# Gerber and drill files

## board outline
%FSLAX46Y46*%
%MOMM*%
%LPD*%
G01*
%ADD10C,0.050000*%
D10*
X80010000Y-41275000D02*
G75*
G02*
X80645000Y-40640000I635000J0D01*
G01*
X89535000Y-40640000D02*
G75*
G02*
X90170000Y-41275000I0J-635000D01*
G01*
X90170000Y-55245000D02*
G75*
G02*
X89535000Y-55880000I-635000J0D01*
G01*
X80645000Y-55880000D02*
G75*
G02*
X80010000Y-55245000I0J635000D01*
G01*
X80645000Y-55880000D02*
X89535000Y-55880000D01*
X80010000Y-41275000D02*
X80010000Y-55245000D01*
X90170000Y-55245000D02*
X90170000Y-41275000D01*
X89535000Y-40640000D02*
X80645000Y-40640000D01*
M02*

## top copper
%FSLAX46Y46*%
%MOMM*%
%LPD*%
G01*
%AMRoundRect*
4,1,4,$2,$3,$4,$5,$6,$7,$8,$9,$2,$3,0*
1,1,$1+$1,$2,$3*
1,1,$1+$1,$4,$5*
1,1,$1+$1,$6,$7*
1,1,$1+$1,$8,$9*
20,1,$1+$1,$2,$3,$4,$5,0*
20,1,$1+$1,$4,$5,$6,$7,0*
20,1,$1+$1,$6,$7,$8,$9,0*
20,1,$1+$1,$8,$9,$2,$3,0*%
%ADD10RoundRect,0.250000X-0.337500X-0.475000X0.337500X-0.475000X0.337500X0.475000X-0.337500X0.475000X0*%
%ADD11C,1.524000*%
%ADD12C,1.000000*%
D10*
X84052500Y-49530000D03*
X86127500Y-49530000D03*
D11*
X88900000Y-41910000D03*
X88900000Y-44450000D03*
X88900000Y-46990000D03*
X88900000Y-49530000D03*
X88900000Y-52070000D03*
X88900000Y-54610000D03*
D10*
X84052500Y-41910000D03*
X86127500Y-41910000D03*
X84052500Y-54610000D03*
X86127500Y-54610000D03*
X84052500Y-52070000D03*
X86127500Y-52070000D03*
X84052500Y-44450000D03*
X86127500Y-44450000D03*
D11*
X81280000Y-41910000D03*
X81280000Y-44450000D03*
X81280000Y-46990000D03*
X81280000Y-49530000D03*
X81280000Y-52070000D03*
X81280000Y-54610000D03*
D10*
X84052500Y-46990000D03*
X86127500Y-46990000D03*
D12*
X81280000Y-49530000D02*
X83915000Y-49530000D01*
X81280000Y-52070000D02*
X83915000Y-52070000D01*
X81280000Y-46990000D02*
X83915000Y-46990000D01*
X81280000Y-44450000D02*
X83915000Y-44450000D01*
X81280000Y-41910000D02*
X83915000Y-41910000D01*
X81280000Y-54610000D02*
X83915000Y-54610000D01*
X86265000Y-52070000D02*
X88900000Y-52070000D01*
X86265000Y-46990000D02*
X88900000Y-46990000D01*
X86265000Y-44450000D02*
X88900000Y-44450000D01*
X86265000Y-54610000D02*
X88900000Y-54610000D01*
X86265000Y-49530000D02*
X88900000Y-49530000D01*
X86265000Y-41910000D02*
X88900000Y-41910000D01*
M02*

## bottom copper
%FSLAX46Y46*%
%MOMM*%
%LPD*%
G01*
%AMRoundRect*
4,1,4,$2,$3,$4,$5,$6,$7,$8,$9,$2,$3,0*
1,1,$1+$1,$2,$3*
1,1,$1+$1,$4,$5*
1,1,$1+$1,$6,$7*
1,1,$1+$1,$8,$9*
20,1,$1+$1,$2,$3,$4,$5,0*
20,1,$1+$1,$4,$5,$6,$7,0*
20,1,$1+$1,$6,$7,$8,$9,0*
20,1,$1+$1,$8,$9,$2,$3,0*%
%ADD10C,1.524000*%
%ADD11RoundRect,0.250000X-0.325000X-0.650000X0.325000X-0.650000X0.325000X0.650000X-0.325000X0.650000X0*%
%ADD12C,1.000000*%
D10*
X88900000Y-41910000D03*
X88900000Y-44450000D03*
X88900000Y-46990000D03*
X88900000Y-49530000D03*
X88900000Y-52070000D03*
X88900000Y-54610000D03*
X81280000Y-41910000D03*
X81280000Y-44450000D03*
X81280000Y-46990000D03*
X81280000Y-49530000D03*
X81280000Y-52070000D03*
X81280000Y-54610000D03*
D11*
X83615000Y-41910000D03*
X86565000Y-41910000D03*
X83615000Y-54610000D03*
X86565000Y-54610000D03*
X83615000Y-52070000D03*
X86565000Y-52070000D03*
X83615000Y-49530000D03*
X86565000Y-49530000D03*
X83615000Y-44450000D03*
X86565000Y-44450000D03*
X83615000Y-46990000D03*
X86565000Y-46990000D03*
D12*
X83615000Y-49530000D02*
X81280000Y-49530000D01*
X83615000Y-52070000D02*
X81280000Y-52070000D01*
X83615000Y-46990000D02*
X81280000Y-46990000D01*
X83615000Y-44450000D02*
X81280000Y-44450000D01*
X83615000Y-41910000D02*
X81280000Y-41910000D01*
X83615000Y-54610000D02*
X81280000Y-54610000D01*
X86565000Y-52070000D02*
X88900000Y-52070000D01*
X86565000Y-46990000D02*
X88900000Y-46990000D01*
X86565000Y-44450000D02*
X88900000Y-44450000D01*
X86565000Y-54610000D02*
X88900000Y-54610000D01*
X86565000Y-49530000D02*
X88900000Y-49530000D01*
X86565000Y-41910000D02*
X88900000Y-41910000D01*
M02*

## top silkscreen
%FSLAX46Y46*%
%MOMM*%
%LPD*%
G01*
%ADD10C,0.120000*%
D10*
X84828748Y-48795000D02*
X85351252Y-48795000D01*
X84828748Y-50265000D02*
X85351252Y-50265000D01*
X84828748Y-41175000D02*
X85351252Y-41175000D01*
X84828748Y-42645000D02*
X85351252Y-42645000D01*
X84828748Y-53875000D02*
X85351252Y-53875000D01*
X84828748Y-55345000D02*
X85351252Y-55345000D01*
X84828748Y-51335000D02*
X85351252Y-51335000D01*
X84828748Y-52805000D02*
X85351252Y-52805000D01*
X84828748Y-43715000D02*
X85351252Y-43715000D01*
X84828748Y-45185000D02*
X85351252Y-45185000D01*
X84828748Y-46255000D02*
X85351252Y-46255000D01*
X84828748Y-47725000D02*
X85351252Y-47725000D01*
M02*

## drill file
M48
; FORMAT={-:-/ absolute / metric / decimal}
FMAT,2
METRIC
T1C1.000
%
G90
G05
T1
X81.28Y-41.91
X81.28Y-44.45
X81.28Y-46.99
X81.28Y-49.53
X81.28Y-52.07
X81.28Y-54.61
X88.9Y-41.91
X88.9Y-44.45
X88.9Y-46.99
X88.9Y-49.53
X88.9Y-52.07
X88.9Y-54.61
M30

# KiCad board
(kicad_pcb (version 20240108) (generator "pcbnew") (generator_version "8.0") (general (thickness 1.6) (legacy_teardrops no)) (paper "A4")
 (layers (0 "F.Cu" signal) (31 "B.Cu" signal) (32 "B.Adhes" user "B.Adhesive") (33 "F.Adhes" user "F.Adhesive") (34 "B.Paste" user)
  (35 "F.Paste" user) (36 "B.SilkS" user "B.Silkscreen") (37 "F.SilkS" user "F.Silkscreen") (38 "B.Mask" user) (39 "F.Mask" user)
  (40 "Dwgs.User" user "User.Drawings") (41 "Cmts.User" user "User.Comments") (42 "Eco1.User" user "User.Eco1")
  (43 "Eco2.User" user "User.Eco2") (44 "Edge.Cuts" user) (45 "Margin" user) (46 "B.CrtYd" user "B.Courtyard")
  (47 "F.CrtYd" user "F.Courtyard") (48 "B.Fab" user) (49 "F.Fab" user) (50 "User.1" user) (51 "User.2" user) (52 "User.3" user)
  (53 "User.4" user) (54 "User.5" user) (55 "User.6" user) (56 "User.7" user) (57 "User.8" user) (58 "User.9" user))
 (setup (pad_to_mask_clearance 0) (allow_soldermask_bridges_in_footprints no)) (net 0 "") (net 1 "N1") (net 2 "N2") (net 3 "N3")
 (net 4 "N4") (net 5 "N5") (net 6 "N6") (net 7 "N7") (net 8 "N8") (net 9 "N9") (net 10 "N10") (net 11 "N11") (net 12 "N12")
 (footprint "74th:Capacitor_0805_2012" (layer "F.Cu") (at 85.09 49.53)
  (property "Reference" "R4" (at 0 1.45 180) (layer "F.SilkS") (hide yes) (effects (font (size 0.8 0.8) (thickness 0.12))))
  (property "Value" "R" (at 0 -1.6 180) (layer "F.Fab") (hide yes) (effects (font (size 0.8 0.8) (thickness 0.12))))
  (fp_line (start -0.261252 -0.735) (end 0.261252 -0.735) (stroke (width 0.12) (type solid)) (layer "F.SilkS"))
  (fp_line (start -0.261252 0.735) (end 0.261252 0.735) (stroke (width 0.12) (type solid)) (layer "F.SilkS"))
  (pad "1" smd roundrect (at -1.0375 0) (size 1.175 1.45) (layers "F.Cu" "F.Paste" "F.Mask") (roundrect_rratio 0.212766) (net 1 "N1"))
  (pad "2" smd roundrect (at 1.0375 0) (size 1.175 1.45) (layers "F.Cu" "F.Paste" "F.Mask") (roundrect_rratio 0.212766) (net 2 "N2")))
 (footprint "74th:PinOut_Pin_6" (layer "F.Cu") (at 88.9 41.91 -90)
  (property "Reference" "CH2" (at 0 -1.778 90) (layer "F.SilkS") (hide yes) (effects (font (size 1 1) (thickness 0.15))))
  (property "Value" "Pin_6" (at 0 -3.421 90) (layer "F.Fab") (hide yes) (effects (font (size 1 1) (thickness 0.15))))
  (pad "1" thru_hole circle (at 0 0 270) (size 1.524 1.524) (drill 1) (layers "*.Cu" "*.Mask") (remove_unused_layers no) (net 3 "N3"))
  (pad "2" thru_hole circle (at 2.54 0 270) (size 1.524 1.524) (drill 1) (layers "*.Cu" "*.Mask") (remove_unused_layers no) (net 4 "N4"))
  (pad "3" thru_hole circle (at 5.08 0 270) (size 1.524 1.524) (drill 1) (layers "*.Cu" "*.Mask") (remove_unused_layers no) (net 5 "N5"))
  (pad "4" thru_hole circle (at 7.62 0 270) (size 1.524 1.524) (drill 1) (layers "*.Cu" "*.Mask") (remove_unused_layers no) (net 2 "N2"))
  (pad "5" thru_hole circle (at 10.16 0 270) (size 1.524 1.524) (drill 1) (layers "*.Cu" "*.Mask") (remove_unused_layers no) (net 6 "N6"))
  (pad "6" thru_hole circle (at 12.7 0 270) (size 1.524 1.524) (drill 1) (layers "*.Cu" "*.Mask") (remove_unused_layers no) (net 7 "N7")))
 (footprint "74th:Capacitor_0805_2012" (layer "F.Cu") (at 85.09 41.91)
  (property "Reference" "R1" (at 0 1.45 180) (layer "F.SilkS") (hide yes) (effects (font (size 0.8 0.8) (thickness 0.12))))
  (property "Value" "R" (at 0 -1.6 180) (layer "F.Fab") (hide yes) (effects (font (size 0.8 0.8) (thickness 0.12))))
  (fp_line (start -0.261252 -0.735) (end 0.261252 -0.735) (stroke (width 0.12) (type solid)) (layer "F.SilkS"))
  (fp_line (start -0.261252 0.735) (end 0.261252 0.735) (stroke (width 0.12) (type solid)) (layer "F.SilkS"))
  (pad "1" smd roundrect (at -1.0375 0) (size 1.175 1.45) (layers "F.Cu" "F.Paste" "F.Mask") (roundrect_rratio 0.212766) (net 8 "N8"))
  (pad "2" smd roundrect (at 1.0375 0) (size 1.175 1.45) (layers "F.Cu" "F.Paste" "F.Mask") (roundrect_rratio 0.212766) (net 3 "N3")))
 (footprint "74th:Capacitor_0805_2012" (layer "F.Cu") (at 85.09 54.61)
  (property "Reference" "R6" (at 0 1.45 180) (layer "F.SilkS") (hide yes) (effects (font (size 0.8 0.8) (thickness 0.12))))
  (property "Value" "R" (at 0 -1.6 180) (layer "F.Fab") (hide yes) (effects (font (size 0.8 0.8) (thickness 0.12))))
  (fp_line (start -0.261252 -0.735) (end 0.261252 -0.735) (stroke (width 0.12) (type solid)) (layer "F.SilkS"))
  (fp_line (start -0.261252 0.735) (end 0.261252 0.735) (stroke (width 0.12) (type solid)) (layer "F.SilkS"))
  (pad "1" smd roundrect (at -1.0375 0) (size 1.175 1.45) (layers "F.Cu" "F.Paste" "F.Mask") (roundrect_rratio 0.212766) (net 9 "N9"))
  (pad "2" smd roundrect (at 1.0375 0) (size 1.175 1.45) (layers "F.Cu" "F.Paste" "F.Mask") (roundrect_rratio 0.212766) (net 7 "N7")))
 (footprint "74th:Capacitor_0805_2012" (layer "F.Cu") (at 85.09 52.07)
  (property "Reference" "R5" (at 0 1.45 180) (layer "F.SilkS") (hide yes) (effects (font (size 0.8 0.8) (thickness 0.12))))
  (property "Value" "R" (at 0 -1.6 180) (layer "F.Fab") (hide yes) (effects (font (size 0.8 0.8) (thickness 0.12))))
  (fp_line (start -0.261252 -0.735) (end 0.261252 -0.735) (stroke (width 0.12) (type solid)) (layer "F.SilkS"))
  (fp_line (start -0.261252 0.735) (end 0.261252 0.735) (stroke (width 0.12) (type solid)) (layer "F.SilkS"))
  (pad "1" smd roundrect (at -1.0375 0) (size 1.175 1.45) (layers "F.Cu" "F.Paste" "F.Mask") (roundrect_rratio 0.212766) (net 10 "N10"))
  (pad "2" smd roundrect (at 1.0375 0) (size 1.175 1.45) (layers "F.Cu" "F.Paste" "F.Mask") (roundrect_rratio 0.212766) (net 6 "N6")))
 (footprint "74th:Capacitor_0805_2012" (layer "F.Cu") (at 85.09 44.45)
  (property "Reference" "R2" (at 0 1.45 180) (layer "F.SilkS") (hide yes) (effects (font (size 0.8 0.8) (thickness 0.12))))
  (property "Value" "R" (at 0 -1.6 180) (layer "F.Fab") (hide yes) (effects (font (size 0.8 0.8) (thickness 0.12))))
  (fp_line (start -0.261252 -0.735) (end 0.261252 -0.735) (stroke (width 0.12) (type solid)) (layer "F.SilkS"))
  (fp_line (start -0.261252 0.735) (end 0.261252 0.735) (stroke (width 0.12) (type solid)) (layer "F.SilkS"))
  (pad "1" smd roundrect (at -1.0375 0) (size 1.175 1.45) (layers "F.Cu" "F.Paste" "F.Mask") (roundrect_rratio 0.212766) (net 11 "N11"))
  (pad "2" smd roundrect (at 1.0375 0) (size 1.175 1.45) (layers "F.Cu" "F.Paste" "F.Mask") (roundrect_rratio 0.212766) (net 4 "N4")))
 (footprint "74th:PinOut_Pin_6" (layer "F.Cu") (at 81.28 41.91 -90)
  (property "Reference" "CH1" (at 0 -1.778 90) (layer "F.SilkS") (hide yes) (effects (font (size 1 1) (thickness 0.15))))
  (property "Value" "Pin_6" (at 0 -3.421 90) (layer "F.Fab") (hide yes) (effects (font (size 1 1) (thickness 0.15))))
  (pad "1" thru_hole circle (at 0 0 270) (size 1.524 1.524) (drill 1) (layers "*.Cu" "*.Mask") (remove_unused_layers no) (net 8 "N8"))
  (pad "2" thru_hole circle (at 2.54 0 270) (size 1.524 1.524) (drill 1) (layers "*.Cu" "*.Mask") (remove_unused_layers no) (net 11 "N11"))
  (pad "3" thru_hole circle (at 5.08 0 270) (size 1.524 1.524) (drill 1) (layers "*.Cu" "*.Mask") (remove_unused_layers no) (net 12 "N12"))
  (pad "4" thru_hole circle (at 7.62 0 270) (size 1.524 1.524) (drill 1) (layers "*.Cu" "*.Mask") (remove_unused_layers no) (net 1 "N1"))
  (pad "5" thru_hole circle (at 10.16 0 270) (size 1.524 1.524) (drill 1) (layers "*.Cu" "*.Mask") (remove_unused_layers no) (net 10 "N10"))
  (pad "6" thru_hole circle (at 12.7 0 270) (size 1.524 1.524) (drill 1) (layers "*.Cu" "*.Mask") (remove_unused_layers no) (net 9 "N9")))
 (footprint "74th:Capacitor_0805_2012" (layer "F.Cu") (at 85.09 46.99)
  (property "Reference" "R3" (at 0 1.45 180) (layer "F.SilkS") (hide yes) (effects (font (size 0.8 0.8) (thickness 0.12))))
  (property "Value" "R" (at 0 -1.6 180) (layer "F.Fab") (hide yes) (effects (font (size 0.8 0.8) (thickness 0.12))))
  (fp_line (start -0.261252 -0.735) (end 0.261252 -0.735) (stroke (width 0.12) (type solid)) (layer "F.SilkS"))
  (fp_line (start -0.261252 0.735) (end 0.261252 0.735) (stroke (width 0.12) (type solid)) (layer "F.SilkS"))
  (pad "1" smd roundrect (at -1.0375 0) (size 1.175 1.45) (layers "F.Cu" "F.Paste" "F.Mask") (roundrect_rratio 0.212766) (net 12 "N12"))
  (pad "2" smd roundrect (at 1.0375 0) (size 1.175 1.45) (layers "F.Cu" "F.Paste" "F.Mask") (roundrect_rratio 0.212766) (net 5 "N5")))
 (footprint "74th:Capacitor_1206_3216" (layer "B.Cu") (at 85.09 41.91)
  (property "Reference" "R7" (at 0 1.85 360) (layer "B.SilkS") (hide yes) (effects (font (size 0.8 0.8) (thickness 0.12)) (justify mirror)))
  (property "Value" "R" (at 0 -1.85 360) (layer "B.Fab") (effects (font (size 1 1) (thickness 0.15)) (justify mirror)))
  (pad "1" smd roundrect (at -1.475 0) (size 1.15 1.8) (layers "B.Cu" "B.Paste" "B.Mask") (roundrect_rratio 0.217391) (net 8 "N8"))
  (pad "2" smd roundrect (at 1.475 0) (size 1.15 1.8) (layers "B.Cu" "B.Paste" "B.Mask") (roundrect_rratio 0.217391) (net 3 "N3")))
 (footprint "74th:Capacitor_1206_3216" (layer "B.Cu") (at 85.09 54.61)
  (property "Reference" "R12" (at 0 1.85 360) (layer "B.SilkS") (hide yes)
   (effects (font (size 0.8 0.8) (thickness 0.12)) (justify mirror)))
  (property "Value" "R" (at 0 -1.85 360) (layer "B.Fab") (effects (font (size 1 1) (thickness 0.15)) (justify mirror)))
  (pad "1" smd roundrect (at -1.475 0) (size 1.15 1.8) (layers "B.Cu" "B.Paste" "B.Mask") (roundrect_rratio 0.217391) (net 9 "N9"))
  (pad "2" smd roundrect (at 1.475 0) (size 1.15 1.8) (layers "B.Cu" "B.Paste" "B.Mask") (roundrect_rratio 0.217391) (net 7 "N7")))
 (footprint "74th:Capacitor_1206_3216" (layer "B.Cu") (at 85.09 52.07)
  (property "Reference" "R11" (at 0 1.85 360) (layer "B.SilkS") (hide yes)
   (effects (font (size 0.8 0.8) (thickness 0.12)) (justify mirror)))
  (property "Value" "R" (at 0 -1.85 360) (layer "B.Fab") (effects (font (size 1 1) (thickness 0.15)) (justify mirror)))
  (pad "1" smd roundrect (at -1.475 0) (size 1.15 1.8) (layers "B.Cu" "B.Paste" "B.Mask") (roundrect_rratio 0.217391) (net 10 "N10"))
  (pad "2" smd roundrect (at 1.475 0) (size 1.15 1.8) (layers "B.Cu" "B.Paste" "B.Mask") (roundrect_rratio 0.217391) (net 6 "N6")))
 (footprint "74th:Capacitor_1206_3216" (layer "B.Cu") (at 85.09 49.53)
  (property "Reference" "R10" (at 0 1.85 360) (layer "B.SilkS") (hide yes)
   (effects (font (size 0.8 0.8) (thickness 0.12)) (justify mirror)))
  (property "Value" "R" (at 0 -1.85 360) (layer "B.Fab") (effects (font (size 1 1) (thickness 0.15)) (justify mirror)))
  (pad "1" smd roundrect (at -1.475 0) (size 1.15 1.8) (layers "B.Cu" "B.Paste" "B.Mask") (roundrect_rratio 0.217391) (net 1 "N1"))
  (pad "2" smd roundrect (at 1.475 0) (size 1.15 1.8) (layers "B.Cu" "B.Paste" "B.Mask") (roundrect_rratio 0.217391) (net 2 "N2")))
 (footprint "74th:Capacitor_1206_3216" (layer "B.Cu") (at 85.09 44.45)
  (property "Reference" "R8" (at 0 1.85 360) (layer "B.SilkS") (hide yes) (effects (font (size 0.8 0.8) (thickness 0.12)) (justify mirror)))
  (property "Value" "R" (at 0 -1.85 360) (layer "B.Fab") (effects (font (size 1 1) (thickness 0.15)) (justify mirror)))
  (pad "1" smd roundrect (at -1.475 0) (size 1.15 1.8) (layers "B.Cu" "B.Paste" "B.Mask") (roundrect_rratio 0.217391) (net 11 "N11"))
  (pad "2" smd roundrect (at 1.475 0) (size 1.15 1.8) (layers "B.Cu" "B.Paste" "B.Mask") (roundrect_rratio 0.217391) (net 4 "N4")))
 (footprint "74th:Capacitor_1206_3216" (layer "B.Cu") (at 85.09 46.99)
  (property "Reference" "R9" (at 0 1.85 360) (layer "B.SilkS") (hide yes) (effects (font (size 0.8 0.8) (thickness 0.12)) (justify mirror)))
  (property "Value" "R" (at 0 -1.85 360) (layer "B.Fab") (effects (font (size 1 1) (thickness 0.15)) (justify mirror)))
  (pad "1" smd roundrect (at -1.475 0) (size 1.15 1.8) (layers "B.Cu" "B.Paste" "B.Mask") (roundrect_rratio 0.217391) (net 12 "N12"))
  (pad "2" smd roundrect (at 1.475 0) (size 1.15 1.8) (layers "B.Cu" "B.Paste" "B.Mask") (roundrect_rratio 0.217391) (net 5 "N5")))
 (gr_arc (start 80.01 41.275) (mid 80.195987 40.825987) (end 80.645 40.64) (stroke (width 0.05) (type default)) (layer "Edge.Cuts"))
 (gr_arc (start 89.535 40.64) (mid 89.984013 40.825987) (end 90.17 41.275) (stroke (width 0.05) (type default)) (layer "Edge.Cuts"))
 (gr_arc (start 90.17 55.245) (mid 89.984013 55.694013) (end 89.535 55.88) (stroke (width 0.05) (type default)) (layer "Edge.Cuts"))
 (gr_arc (start 80.645 55.88) (mid 80.195987 55.694013) (end 80.01 55.245) (stroke (width 0.05) (type default)) (layer "Edge.Cuts"))
 (gr_line (start 80.645 55.88) (end 89.535 55.88) (stroke (width 0.05) (type default)) (layer "Edge.Cuts"))
 (gr_line (start 80.01 41.275) (end 80.01 55.245) (stroke (width 0.05) (type default)) (layer "Edge.Cuts"))
 (gr_line (start 90.17 55.245) (end 90.17 41.275) (stroke (width 0.05) (type default)) (layer "Edge.Cuts"))
 (gr_line (start 89.535 40.64) (end 80.645 40.64) (stroke (width 0.05) (type default)) (layer "Edge.Cuts"))
 (segment (start 81.28 49.53) (end 83.915 49.53) (width 1) (layer "F.Cu") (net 1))
 (segment (start 83.615 49.53) (end 81.28 49.53) (width 1) (layer "B.Cu") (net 1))
 (segment (start 81.28 52.07) (end 83.915 52.07) (width 1) (layer "F.Cu") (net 10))
 (segment (start 83.615 52.07) (end 81.28 52.07) (width 1) (layer "B.Cu") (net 10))
 (segment (start 81.28 46.99) (end 83.915 46.99) (width 1) (layer "F.Cu") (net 12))
 (segment (start 83.615 46.99) (end 81.28 46.99) (width 1) (layer "B.Cu") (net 12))
 (segment (start 81.28 44.45) (end 83.915 44.45) (width 1) (layer "F.Cu") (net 11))
 (segment (start 83.615 44.45) (end 81.28 44.45) (width 1) (layer "B.Cu") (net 11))
 (segment (start 81.28 41.91) (end 83.915 41.91) (width 1) (layer "F.Cu") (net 8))
 (segment (start 83.615 41.91) (end 81.28 41.91) (width 1) (layer "B.Cu") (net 8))
 (segment (start 81.28 54.61) (end 83.915 54.61) (width 1) (layer "F.Cu") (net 9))
 (segment (start 83.615 54.61) (end 81.28 54.61) (width 1) (layer "B.Cu") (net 9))
 (segment (start 86.265 52.07) (end 88.9 52.07) (width 1) (layer "F.Cu") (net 6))
 (segment (start 86.565 52.07) (end 88.9 52.07) (width 1) (layer "B.Cu") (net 6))
 (segment (start 86.265 46.99) (end 88.9 46.99) (width 1) (layer "F.Cu") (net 5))
 (segment (start 86.565 46.99) (end 88.9 46.99) (width 1) (layer "B.Cu") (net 5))
 (segment (start 86.265 44.45) (end 88.9 44.45) (width 1) (layer "F.Cu") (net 4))
 (segment (start 86.565 44.45) (end 88.9 44.45) (width 1) (layer "B.Cu") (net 4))
 (segment (start 86.265 54.61) (end 88.9 54.61) (width 1) (layer "F.Cu") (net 7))
 (segment (start 86.565 54.61) (end 88.9 54.61) (width 1) (layer "B.Cu") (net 7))
 (segment (start 86.265 49.53) (end 88.9 49.53) (width 1) (layer "F.Cu") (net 2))
 (segment (start 86.565 49.53) (end 88.9 49.53) (width 1) (layer "B.Cu") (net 2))
 (segment (start 86.265 41.91) (end 88.9 41.91) (width 1) (layer "F.Cu") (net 3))
 (segment (start 86.565 41.91) (end 88.9 41.91) (width 1) (layer "B.Cu") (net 3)))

